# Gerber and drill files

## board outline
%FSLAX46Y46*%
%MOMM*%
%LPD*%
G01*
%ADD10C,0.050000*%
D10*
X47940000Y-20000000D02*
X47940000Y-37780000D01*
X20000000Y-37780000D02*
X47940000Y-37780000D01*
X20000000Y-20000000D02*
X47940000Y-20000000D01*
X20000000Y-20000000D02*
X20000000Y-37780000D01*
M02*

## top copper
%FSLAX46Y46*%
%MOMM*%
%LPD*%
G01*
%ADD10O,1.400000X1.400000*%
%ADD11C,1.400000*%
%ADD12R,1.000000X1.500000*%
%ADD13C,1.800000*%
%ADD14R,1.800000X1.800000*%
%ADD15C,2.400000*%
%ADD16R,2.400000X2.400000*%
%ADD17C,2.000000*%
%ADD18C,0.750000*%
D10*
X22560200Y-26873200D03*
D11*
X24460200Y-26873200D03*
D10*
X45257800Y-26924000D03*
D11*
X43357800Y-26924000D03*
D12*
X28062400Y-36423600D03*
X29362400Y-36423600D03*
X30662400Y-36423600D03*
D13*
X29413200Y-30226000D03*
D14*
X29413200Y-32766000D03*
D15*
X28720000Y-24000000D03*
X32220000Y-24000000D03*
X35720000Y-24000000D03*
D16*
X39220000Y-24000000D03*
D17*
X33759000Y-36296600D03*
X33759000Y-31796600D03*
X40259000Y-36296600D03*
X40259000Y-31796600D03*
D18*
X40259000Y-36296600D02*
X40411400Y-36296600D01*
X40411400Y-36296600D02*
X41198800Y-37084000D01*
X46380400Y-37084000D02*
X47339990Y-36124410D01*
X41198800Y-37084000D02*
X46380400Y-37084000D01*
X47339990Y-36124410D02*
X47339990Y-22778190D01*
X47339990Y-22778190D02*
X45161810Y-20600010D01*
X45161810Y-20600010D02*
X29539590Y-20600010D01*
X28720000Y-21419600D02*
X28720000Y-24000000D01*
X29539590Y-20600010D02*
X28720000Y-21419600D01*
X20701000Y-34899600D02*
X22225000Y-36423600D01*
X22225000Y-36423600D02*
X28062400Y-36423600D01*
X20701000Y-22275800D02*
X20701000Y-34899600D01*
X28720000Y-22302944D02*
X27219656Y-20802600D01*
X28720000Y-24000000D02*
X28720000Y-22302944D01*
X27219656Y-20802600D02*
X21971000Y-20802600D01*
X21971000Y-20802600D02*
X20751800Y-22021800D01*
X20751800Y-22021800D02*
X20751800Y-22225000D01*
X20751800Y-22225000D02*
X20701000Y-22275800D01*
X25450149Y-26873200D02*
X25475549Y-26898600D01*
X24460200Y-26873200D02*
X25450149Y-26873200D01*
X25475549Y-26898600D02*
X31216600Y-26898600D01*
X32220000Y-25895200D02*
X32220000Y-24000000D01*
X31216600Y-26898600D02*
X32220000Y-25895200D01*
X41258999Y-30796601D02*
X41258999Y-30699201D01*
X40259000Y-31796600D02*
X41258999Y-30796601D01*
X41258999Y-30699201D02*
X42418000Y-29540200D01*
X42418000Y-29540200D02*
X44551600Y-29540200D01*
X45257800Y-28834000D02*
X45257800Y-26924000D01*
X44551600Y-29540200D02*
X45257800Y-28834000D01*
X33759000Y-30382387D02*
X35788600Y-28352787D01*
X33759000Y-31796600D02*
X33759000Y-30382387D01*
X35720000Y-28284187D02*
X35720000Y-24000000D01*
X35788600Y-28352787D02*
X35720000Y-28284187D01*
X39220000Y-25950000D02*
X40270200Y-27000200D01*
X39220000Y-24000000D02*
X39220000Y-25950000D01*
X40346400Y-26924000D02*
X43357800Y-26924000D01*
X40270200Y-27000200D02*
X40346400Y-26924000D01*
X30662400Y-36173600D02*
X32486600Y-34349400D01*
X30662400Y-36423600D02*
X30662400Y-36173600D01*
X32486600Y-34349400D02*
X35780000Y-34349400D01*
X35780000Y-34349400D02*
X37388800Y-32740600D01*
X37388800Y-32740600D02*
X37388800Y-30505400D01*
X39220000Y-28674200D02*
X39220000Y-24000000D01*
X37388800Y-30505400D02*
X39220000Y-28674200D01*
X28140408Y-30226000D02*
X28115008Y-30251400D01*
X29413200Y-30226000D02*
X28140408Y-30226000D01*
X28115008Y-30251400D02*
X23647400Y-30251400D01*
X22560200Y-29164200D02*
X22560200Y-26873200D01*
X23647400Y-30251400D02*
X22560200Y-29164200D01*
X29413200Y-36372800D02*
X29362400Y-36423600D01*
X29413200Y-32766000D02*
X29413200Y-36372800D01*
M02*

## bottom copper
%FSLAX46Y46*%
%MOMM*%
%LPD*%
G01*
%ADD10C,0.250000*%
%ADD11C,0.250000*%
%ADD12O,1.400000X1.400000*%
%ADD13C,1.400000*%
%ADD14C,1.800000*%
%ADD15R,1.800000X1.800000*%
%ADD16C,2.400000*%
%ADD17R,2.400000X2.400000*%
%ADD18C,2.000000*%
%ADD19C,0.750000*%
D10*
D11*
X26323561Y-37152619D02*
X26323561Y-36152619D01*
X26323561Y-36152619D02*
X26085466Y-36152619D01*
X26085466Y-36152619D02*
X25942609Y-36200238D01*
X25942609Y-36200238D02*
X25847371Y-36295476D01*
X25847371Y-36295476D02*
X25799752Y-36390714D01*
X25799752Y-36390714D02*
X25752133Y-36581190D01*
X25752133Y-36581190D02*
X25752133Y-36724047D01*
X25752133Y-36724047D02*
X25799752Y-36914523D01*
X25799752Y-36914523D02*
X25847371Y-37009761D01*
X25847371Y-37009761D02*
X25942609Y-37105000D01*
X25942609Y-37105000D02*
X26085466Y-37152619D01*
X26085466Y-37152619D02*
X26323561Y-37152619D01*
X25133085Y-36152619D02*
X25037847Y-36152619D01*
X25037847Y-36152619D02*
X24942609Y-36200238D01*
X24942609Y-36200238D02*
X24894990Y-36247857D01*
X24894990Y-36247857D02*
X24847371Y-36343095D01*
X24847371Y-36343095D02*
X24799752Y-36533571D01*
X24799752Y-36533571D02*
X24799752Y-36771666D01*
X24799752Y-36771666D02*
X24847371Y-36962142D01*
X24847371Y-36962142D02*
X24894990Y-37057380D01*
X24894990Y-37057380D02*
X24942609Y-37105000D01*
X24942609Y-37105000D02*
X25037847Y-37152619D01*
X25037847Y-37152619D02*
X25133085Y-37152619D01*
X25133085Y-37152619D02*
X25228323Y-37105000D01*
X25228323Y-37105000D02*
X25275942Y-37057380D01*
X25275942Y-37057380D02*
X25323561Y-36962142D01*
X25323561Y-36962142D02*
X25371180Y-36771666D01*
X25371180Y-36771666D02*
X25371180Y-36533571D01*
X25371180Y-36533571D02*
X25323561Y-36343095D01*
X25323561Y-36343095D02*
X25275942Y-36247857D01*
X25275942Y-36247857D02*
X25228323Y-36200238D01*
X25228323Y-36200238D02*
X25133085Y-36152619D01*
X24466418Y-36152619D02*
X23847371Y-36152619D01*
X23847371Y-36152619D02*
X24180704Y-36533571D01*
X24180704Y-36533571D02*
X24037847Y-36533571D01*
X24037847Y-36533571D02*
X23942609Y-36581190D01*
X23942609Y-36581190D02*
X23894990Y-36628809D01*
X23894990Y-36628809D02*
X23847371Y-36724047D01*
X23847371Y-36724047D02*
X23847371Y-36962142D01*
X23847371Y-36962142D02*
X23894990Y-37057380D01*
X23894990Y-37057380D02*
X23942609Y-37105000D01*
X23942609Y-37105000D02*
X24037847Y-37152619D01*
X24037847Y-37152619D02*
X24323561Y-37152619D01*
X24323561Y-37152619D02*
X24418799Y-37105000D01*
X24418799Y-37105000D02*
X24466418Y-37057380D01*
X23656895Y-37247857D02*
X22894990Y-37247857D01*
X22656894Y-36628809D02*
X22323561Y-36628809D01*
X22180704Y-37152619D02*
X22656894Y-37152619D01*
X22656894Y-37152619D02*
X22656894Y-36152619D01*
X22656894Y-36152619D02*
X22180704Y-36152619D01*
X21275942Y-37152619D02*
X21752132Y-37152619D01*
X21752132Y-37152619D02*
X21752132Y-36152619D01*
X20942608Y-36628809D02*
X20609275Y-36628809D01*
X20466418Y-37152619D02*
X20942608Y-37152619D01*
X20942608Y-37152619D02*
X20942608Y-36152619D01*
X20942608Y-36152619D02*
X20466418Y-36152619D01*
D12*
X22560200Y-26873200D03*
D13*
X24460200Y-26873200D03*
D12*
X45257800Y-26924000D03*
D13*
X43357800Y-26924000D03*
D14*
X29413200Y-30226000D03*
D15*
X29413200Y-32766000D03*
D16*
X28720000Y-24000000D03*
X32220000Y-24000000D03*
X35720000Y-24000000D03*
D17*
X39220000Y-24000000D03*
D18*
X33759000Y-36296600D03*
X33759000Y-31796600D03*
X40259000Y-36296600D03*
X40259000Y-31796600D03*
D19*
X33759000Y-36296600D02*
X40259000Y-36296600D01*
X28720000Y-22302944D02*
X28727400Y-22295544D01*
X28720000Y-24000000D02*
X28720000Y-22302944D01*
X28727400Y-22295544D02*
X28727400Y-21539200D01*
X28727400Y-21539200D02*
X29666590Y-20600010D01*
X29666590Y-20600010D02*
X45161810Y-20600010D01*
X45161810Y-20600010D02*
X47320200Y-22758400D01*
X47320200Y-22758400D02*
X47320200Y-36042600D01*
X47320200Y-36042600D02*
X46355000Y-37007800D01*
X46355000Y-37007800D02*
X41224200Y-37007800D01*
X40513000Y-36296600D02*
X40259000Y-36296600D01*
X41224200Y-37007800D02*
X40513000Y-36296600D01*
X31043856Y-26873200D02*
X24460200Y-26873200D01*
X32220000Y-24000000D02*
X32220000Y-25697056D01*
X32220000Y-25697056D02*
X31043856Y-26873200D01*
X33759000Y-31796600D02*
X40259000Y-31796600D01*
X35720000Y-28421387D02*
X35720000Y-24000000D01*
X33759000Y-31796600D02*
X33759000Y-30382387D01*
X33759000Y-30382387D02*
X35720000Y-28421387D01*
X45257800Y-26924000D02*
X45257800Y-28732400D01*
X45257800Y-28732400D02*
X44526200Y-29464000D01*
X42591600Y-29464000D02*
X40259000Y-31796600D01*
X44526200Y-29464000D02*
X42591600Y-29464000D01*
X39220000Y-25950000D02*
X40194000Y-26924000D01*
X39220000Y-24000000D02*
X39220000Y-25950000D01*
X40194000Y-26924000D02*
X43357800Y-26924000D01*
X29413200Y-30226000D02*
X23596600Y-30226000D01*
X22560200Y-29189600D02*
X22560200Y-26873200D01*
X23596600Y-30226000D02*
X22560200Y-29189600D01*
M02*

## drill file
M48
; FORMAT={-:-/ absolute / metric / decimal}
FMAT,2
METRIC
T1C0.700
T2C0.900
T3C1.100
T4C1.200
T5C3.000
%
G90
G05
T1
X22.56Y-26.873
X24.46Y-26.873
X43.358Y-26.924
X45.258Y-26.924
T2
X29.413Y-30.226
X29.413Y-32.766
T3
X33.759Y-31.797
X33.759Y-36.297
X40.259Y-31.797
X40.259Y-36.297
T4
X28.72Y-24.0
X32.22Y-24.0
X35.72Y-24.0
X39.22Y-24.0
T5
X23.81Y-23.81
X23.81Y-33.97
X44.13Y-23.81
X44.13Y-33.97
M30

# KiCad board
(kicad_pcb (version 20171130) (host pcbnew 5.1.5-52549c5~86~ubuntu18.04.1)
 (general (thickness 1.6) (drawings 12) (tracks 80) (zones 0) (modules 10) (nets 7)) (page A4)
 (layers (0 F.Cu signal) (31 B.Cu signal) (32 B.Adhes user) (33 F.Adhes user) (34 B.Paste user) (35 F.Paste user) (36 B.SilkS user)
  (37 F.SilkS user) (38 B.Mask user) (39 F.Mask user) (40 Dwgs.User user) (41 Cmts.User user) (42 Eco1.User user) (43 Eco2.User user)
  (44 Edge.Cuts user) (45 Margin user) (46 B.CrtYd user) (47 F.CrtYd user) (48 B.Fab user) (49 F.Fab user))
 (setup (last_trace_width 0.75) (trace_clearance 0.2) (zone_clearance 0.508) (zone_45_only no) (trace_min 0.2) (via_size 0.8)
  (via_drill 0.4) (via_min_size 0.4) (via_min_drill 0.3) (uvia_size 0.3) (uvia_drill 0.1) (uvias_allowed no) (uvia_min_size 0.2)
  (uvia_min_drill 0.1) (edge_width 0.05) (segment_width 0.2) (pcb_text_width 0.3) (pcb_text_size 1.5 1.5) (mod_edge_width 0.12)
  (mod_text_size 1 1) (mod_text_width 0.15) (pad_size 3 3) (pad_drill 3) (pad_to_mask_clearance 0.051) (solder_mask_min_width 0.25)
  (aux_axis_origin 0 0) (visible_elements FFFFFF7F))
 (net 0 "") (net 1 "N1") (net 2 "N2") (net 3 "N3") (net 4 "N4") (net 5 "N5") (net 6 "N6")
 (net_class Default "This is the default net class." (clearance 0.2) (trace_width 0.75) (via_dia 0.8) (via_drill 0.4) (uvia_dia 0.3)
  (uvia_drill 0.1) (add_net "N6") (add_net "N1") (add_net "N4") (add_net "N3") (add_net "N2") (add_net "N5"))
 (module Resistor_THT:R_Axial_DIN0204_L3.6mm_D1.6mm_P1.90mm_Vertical (layer F.Cu) (at 24.4602 26.8732 180)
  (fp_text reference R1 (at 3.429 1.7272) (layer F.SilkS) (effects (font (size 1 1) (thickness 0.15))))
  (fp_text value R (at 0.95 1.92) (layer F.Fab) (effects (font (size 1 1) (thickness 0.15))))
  (pad 2 thru_hole oval (at 1.9 0 180) (size 1.4 1.4) (drill 0.7) (layers *.Cu *.Mask) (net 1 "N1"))
  (pad 1 thru_hole circle (at 0 0 180) (size 1.4 1.4) (drill 0.7) (layers *.Cu *.Mask) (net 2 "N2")))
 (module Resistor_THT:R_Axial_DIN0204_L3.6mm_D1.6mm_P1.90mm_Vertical (layer F.Cu) (at 43.3578 26.924)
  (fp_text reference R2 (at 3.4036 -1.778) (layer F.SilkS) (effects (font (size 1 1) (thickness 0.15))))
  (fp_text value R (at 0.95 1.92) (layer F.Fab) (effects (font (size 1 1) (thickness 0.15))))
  (pad 2 thru_hole oval (at 1.9 0) (size 1.4 1.4) (drill 0.7) (layers *.Cu *.Mask) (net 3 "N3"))
  (pad 1 thru_hole circle (at 0 0) (size 1.4 1.4) (drill 0.7) (layers *.Cu *.Mask) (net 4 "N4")))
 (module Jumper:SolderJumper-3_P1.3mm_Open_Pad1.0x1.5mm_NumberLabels (layer F.Cu) (at 29.3624 36.4236)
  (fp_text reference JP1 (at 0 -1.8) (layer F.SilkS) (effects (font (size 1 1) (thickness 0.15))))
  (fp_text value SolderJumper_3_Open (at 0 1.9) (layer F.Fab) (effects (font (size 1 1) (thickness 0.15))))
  (pad 1 smd rect (at -1.3 0) (size 1 1.5) (layers F.Cu F.Mask) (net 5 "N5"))
  (pad 2 smd rect (at 0 0) (size 1 1.5) (layers F.Cu F.Mask) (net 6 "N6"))
  (pad 3 smd rect (at 1.3 0) (size 1 1.5) (layers F.Cu F.Mask) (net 4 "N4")))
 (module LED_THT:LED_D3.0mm (layer F.Cu) (at 29.4132 32.766 90)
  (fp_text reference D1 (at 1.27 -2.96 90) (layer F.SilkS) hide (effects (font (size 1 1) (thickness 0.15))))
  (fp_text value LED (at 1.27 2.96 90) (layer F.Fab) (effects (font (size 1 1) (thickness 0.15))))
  (pad 2 thru_hole circle (at 2.54 0 90) (size 1.8 1.8) (drill 0.9) (layers *.Cu *.Mask) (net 1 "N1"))
  (pad 1 thru_hole rect (at 0 0 90) (size 1.8 1.8) (drill 0.9) (layers *.Cu *.Mask) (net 6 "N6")))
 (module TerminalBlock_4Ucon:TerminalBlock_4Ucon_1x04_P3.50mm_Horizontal (layer F.Cu) (at 39.22 24 180)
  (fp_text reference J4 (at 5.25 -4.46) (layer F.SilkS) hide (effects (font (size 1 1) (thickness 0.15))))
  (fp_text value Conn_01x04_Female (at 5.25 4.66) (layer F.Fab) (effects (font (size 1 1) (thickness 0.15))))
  (pad 4 thru_hole circle (at 10.5 0 180) (size 2.4 2.4) (drill 1.2) (layers *.Cu *.Mask) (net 5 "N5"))
  (pad 3 thru_hole circle (at 7 0 180) (size 2.4 2.4) (drill 1.2) (layers *.Cu *.Mask) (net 2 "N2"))
  (pad 2 thru_hole circle (at 3.5 0 180) (size 2.4 2.4) (drill 1.2) (layers *.Cu *.Mask) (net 3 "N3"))
  (pad 1 thru_hole rect (at 0 0 180) (size 2.4 2.4) (drill 1.2) (layers *.Cu *.Mask) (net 4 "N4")))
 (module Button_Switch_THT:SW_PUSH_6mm (layer F.Cu) (at 40.259 36.2966 180)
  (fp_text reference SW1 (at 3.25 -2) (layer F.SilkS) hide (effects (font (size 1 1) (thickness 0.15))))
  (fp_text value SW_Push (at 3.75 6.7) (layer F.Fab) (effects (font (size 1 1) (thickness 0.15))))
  (pad 1 thru_hole circle (at 6.5 0 270) (size 2 2) (drill 1.1) (layers *.Cu *.Mask) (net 5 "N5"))
  (pad 2 thru_hole circle (at 6.5 4.5 270) (size 2 2) (drill 1.1) (layers *.Cu *.Mask) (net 3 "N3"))
  (pad 1 thru_hole circle (at 0 0 270) (size 2 2) (drill 1.1) (layers *.Cu *.Mask) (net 5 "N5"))
  (pad 2 thru_hole circle (at 0 4.5 270) (size 2 2) (drill 1.1) (layers *.Cu *.Mask) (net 3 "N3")))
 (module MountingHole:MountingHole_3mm (layer F.Cu) (at 44.13 33.97)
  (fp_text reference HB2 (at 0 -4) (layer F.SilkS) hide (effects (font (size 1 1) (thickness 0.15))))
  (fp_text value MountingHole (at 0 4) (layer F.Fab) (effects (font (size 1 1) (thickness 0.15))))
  (pad 1 np_thru_hole circle (at 0 0) (size 3 3) (drill 3) (layers *.Cu *.Mask)))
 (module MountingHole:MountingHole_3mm (layer F.Cu) (at 23.81 33.97)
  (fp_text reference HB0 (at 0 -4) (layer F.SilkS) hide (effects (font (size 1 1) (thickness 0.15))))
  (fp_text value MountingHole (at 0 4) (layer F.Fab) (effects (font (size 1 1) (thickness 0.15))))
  (pad 1 np_thru_hole circle (at 0 0) (size 3 3) (drill 3) (layers *.Cu *.Mask)))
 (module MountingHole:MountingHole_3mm (layer F.Cu) (at 44.13 23.81)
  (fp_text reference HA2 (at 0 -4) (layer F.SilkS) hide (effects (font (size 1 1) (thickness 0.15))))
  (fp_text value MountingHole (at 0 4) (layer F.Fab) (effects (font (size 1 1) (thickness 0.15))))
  (pad 1 np_thru_hole circle (at 0 0) (size 3 3) (drill 3) (layers *.Cu *.Mask)))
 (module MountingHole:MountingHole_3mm (layer F.Cu) (at 23.81 23.81)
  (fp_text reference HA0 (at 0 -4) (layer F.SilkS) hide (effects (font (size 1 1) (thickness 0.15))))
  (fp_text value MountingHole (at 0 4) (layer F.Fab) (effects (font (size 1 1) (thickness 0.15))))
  (pad 1 np_thru_hole circle (at 0 0) (size 3 3) (drill 3) (layers *.Cu *.Mask)))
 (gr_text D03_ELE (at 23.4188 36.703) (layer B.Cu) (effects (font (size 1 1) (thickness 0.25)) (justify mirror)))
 (gr_line (start 47.94 20) (end 47.94 37.78) (layer Edge.Cuts) (width 0.05))
 (gr_line (start 20 37.78) (end 47.94 37.78) (layer Edge.Cuts) (width 0.05))
 (gr_line (start 20 20) (end 47.94 20) (layer Edge.Cuts) (width 0.05))
 (gr_line (start 20 20) (end 20 37.78) (layer Edge.Cuts) (width 0.05))
 (segment (start 40.259 36.2966) (end 40.4114 36.2966) (width 0.75) (layer F.Cu) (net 5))
 (segment (start 40.4114 36.2966) (end 41.1988 37.084) (width 0.75) (layer F.Cu) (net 5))
 (segment (start 46.3804 37.084) (end 47.33999 36.12441) (width 0.75) (layer F.Cu) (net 5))
 (segment (start 41.1988 37.084) (end 46.3804 37.084) (width 0.75) (layer F.Cu) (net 5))
 (segment (start 47.33999 36.12441) (end 47.33999 22.77819) (width 0.75) (layer F.Cu) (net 5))
 (segment (start 47.33999 22.77819) (end 45.16181 20.60001) (width 0.75) (layer F.Cu) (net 5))
 (segment (start 45.16181 20.60001) (end 29.53959 20.60001) (width 0.75) (layer F.Cu) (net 5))
 (segment (start 28.72 21.4196) (end 28.72 24) (width 0.75) (layer F.Cu) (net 5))
 (segment (start 29.53959 20.60001) (end 28.72 21.4196) (width 0.75) (layer F.Cu) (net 5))
 (segment (start 20.701 34.8996) (end 22.225 36.4236) (width 0.75) (layer F.Cu) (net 5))
 (segment (start 22.225 36.4236) (end 28.0624 36.4236) (width 0.75) (layer F.Cu) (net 5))
 (segment (start 20.701 22.2758) (end 20.701 34.8996) (width 0.75) (layer F.Cu) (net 5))
 (segment (start 28.72 22.302944) (end 27.219656 20.8026) (width 0.75) (layer F.Cu) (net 5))
 (segment (start 28.72 24) (end 28.72 22.302944) (width 0.75) (layer F.Cu) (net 5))
 (segment (start 27.219656 20.8026) (end 21.971 20.8026) (width 0.75) (layer F.Cu) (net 5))
 (segment (start 21.971 20.8026) (end 20.7518 22.0218) (width 0.75) (layer F.Cu) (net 5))
 (segment (start 20.7518 22.0218) (end 20.7518 22.225) (width 0.75) (layer F.Cu) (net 5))
 (segment (start 20.7518 22.225) (end 20.701 22.2758) (width 0.75) (layer F.Cu) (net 5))
 (segment (start 33.759 36.2966) (end 40.259 36.2966) (width 0.75) (layer B.Cu) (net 5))
 (segment (start 28.72 22.302944) (end 28.7274 22.295544) (width 0.75) (layer B.Cu) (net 5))
 (segment (start 28.72 24) (end 28.72 22.302944) (width 0.75) (layer B.Cu) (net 5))
 (segment (start 28.7274 22.295544) (end 28.7274 21.5392) (width 0.75) (layer B.Cu) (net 5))
 (segment (start 28.7274 21.5392) (end 29.66659 20.60001) (width 0.75) (layer B.Cu) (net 5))
 (segment (start 29.66659 20.60001) (end 45.16181 20.60001) (width 0.75) (layer B.Cu) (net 5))
 (segment (start 45.16181 20.60001) (end 47.3202 22.7584) (width 0.75) (layer B.Cu) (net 5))
 (segment (start 47.3202 22.7584) (end 47.3202 36.0426) (width 0.75) (layer B.Cu) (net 5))
 (segment (start 47.3202 36.0426) (end 46.355 37.0078) (width 0.75) (layer B.Cu) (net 5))
 (segment (start 46.355 37.0078) (end 41.2242 37.0078) (width 0.75) (layer B.Cu) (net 5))
 (segment (start 40.513 36.2966) (end 40.259 36.2966) (width 0.75) (layer B.Cu) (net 5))
 (segment (start 41.2242 37.0078) (end 40.513 36.2966) (width 0.75) (layer B.Cu) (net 5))
 (segment (start 25.450149 26.8732) (end 25.475549 26.8986) (width 0.75) (layer F.Cu) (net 2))
 (segment (start 24.4602 26.8732) (end 25.450149 26.8732) (width 0.75) (layer F.Cu) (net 2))
 (segment (start 25.475549 26.8986) (end 31.2166 26.8986) (width 0.75) (layer F.Cu) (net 2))
 (segment (start 32.22 25.8952) (end 32.22 24) (width 0.75) (layer F.Cu) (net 2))
 (segment (start 31.2166 26.8986) (end 32.22 25.8952) (width 0.75) (layer F.Cu) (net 2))
 (segment (start 31.043856 26.8732) (end 24.4602 26.8732) (width 0.75) (layer B.Cu) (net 2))
 (segment (start 32.22 24) (end 32.22 25.697056) (width 0.75) (layer B.Cu) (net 2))
 (segment (start 32.22 25.697056) (end 31.043856 26.8732) (width 0.75) (layer B.Cu) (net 2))
 (segment (start 41.258999 30.796601) (end 41.258999 30.699201) (width 0.75) (layer F.Cu) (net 3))
 (segment (start 40.259 31.7966) (end 41.258999 30.796601) (width 0.75) (layer F.Cu) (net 3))
 (segment (start 41.258999 30.699201) (end 42.418 29.5402) (width 0.75) (layer F.Cu) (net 3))
 (segment (start 42.418 29.5402) (end 44.5516 29.5402) (width 0.75) (layer F.Cu) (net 3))
 (segment (start 45.2578 28.834) (end 45.2578 26.924) (width 0.75) (layer F.Cu) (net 3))
 (segment (start 44.5516 29.5402) (end 45.2578 28.834) (width 0.75) (layer F.Cu) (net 3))
 (segment (start 33.759 30.382387) (end 35.7886 28.352787) (width 0.75) (layer F.Cu) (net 3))
 (segment (start 33.759 31.7966) (end 33.759 30.382387) (width 0.75) (layer F.Cu) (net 3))
 (segment (start 35.72 28.284187) (end 35.72 24) (width 0.75) (layer F.Cu) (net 3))
 (segment (start 35.7886 28.352787) (end 35.72 28.284187) (width 0.75) (layer F.Cu) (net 3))
 (segment (start 33.759 31.7966) (end 40.259 31.7966) (width 0.75) (layer B.Cu) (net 3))
 (segment (start 35.72 28.421387) (end 35.72 24) (width 0.75) (layer B.Cu) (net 3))
 (segment (start 33.759 31.7966) (end 33.759 30.382387) (width 0.75) (layer B.Cu) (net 3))
 (segment (start 33.759 30.382387) (end 35.72 28.421387) (width 0.75) (layer B.Cu) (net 3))
 (segment (start 45.2578 26.924) (end 45.2578 28.7324) (width 0.75) (layer B.Cu) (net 3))
 (segment (start 45.2578 28.7324) (end 44.5262 29.464) (width 0.75) (layer B.Cu) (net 3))
 (segment (start 42.5916 29.464) (end 40.259 31.7966) (width 0.75) (layer B.Cu) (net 3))
 (segment (start 44.5262 29.464) (end 42.5916 29.464) (width 0.75) (layer B.Cu) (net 3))
 (segment (start 39.22 25.95) (end 40.2702 27.0002) (width 0.75) (layer F.Cu) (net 4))
 (segment (start 39.22 24) (end 39.22 25.95) (width 0.75) (layer F.Cu) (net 4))
 (segment (start 40.3464 26.924) (end 43.3578 26.924) (width 0.75) (layer F.Cu) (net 4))
 (segment (start 40.2702 27.0002) (end 40.3464 26.924) (width 0.75) (layer F.Cu) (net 4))
 (segment (start 30.6624 36.1736) (end 32.4866 34.3494) (width 0.75) (layer F.Cu) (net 4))
 (segment (start 30.6624 36.4236) (end 30.6624 36.1736) (width 0.75) (layer F.Cu) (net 4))
 (segment (start 32.4866 34.3494) (end 35.78 34.3494) (width 0.75) (layer F.Cu) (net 4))
 (segment (start 35.78 34.3494) (end 37.3888 32.7406) (width 0.75) (layer F.Cu) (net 4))
 (segment (start 37.3888 32.7406) (end 37.3888 30.5054) (width 0.75) (layer F.Cu) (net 4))
 (segment (start 39.22 28.6742) (end 39.22 24) (width 0.75) (layer F.Cu) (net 4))
 (segment (start 37.3888 30.5054) (end 39.22 28.6742) (width 0.75) (layer F.Cu) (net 4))
 (segment (start 39.22 25.95) (end 40.194 26.924) (width 0.75) (layer B.Cu) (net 4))
 (segment (start 39.22 24) (end 39.22 25.95) (width 0.75) (layer B.Cu) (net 4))
 (segment (start 40.194 26.924) (end 43.3578 26.924) (width 0.75) (layer B.Cu) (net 4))
 (segment (start 28.140408 30.226) (end 28.115008 30.2514) (width 0.75) (layer F.Cu) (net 1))
 (segment (start 29.4132 30.226) (end 28.140408 30.226) (width 0.75) (layer F.Cu) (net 1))
 (segment (start 28.115008 30.2514) (end 23.6474 30.2514) (width 0.75) (layer F.Cu) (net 1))
 (segment (start 22.5602 29.1642) (end 22.5602 26.8732) (width 0.75) (layer F.Cu) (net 1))
 (segment (start 23.6474 30.2514) (end 22.5602 29.1642) (width 0.75) (layer F.Cu) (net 1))
 (segment (start 29.4132 30.226) (end 23.5966 30.226) (width 0.75) (layer B.Cu) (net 1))
 (segment (start 22.5602 29.1896) (end 22.5602 26.8732) (width 0.75) (layer B.Cu) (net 1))
 (segment (start 23.5966 30.226) (end 22.5602 29.1896) (width 0.75) (layer B.Cu) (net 1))
 (segment (start 29.4132 36.3728) (end 29.3624 36.4236) (width 0.75) (layer F.Cu) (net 6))
 (segment (start 29.4132 32.766) (end 29.4132 36.3728) (width 0.75) (layer F.Cu) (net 6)))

